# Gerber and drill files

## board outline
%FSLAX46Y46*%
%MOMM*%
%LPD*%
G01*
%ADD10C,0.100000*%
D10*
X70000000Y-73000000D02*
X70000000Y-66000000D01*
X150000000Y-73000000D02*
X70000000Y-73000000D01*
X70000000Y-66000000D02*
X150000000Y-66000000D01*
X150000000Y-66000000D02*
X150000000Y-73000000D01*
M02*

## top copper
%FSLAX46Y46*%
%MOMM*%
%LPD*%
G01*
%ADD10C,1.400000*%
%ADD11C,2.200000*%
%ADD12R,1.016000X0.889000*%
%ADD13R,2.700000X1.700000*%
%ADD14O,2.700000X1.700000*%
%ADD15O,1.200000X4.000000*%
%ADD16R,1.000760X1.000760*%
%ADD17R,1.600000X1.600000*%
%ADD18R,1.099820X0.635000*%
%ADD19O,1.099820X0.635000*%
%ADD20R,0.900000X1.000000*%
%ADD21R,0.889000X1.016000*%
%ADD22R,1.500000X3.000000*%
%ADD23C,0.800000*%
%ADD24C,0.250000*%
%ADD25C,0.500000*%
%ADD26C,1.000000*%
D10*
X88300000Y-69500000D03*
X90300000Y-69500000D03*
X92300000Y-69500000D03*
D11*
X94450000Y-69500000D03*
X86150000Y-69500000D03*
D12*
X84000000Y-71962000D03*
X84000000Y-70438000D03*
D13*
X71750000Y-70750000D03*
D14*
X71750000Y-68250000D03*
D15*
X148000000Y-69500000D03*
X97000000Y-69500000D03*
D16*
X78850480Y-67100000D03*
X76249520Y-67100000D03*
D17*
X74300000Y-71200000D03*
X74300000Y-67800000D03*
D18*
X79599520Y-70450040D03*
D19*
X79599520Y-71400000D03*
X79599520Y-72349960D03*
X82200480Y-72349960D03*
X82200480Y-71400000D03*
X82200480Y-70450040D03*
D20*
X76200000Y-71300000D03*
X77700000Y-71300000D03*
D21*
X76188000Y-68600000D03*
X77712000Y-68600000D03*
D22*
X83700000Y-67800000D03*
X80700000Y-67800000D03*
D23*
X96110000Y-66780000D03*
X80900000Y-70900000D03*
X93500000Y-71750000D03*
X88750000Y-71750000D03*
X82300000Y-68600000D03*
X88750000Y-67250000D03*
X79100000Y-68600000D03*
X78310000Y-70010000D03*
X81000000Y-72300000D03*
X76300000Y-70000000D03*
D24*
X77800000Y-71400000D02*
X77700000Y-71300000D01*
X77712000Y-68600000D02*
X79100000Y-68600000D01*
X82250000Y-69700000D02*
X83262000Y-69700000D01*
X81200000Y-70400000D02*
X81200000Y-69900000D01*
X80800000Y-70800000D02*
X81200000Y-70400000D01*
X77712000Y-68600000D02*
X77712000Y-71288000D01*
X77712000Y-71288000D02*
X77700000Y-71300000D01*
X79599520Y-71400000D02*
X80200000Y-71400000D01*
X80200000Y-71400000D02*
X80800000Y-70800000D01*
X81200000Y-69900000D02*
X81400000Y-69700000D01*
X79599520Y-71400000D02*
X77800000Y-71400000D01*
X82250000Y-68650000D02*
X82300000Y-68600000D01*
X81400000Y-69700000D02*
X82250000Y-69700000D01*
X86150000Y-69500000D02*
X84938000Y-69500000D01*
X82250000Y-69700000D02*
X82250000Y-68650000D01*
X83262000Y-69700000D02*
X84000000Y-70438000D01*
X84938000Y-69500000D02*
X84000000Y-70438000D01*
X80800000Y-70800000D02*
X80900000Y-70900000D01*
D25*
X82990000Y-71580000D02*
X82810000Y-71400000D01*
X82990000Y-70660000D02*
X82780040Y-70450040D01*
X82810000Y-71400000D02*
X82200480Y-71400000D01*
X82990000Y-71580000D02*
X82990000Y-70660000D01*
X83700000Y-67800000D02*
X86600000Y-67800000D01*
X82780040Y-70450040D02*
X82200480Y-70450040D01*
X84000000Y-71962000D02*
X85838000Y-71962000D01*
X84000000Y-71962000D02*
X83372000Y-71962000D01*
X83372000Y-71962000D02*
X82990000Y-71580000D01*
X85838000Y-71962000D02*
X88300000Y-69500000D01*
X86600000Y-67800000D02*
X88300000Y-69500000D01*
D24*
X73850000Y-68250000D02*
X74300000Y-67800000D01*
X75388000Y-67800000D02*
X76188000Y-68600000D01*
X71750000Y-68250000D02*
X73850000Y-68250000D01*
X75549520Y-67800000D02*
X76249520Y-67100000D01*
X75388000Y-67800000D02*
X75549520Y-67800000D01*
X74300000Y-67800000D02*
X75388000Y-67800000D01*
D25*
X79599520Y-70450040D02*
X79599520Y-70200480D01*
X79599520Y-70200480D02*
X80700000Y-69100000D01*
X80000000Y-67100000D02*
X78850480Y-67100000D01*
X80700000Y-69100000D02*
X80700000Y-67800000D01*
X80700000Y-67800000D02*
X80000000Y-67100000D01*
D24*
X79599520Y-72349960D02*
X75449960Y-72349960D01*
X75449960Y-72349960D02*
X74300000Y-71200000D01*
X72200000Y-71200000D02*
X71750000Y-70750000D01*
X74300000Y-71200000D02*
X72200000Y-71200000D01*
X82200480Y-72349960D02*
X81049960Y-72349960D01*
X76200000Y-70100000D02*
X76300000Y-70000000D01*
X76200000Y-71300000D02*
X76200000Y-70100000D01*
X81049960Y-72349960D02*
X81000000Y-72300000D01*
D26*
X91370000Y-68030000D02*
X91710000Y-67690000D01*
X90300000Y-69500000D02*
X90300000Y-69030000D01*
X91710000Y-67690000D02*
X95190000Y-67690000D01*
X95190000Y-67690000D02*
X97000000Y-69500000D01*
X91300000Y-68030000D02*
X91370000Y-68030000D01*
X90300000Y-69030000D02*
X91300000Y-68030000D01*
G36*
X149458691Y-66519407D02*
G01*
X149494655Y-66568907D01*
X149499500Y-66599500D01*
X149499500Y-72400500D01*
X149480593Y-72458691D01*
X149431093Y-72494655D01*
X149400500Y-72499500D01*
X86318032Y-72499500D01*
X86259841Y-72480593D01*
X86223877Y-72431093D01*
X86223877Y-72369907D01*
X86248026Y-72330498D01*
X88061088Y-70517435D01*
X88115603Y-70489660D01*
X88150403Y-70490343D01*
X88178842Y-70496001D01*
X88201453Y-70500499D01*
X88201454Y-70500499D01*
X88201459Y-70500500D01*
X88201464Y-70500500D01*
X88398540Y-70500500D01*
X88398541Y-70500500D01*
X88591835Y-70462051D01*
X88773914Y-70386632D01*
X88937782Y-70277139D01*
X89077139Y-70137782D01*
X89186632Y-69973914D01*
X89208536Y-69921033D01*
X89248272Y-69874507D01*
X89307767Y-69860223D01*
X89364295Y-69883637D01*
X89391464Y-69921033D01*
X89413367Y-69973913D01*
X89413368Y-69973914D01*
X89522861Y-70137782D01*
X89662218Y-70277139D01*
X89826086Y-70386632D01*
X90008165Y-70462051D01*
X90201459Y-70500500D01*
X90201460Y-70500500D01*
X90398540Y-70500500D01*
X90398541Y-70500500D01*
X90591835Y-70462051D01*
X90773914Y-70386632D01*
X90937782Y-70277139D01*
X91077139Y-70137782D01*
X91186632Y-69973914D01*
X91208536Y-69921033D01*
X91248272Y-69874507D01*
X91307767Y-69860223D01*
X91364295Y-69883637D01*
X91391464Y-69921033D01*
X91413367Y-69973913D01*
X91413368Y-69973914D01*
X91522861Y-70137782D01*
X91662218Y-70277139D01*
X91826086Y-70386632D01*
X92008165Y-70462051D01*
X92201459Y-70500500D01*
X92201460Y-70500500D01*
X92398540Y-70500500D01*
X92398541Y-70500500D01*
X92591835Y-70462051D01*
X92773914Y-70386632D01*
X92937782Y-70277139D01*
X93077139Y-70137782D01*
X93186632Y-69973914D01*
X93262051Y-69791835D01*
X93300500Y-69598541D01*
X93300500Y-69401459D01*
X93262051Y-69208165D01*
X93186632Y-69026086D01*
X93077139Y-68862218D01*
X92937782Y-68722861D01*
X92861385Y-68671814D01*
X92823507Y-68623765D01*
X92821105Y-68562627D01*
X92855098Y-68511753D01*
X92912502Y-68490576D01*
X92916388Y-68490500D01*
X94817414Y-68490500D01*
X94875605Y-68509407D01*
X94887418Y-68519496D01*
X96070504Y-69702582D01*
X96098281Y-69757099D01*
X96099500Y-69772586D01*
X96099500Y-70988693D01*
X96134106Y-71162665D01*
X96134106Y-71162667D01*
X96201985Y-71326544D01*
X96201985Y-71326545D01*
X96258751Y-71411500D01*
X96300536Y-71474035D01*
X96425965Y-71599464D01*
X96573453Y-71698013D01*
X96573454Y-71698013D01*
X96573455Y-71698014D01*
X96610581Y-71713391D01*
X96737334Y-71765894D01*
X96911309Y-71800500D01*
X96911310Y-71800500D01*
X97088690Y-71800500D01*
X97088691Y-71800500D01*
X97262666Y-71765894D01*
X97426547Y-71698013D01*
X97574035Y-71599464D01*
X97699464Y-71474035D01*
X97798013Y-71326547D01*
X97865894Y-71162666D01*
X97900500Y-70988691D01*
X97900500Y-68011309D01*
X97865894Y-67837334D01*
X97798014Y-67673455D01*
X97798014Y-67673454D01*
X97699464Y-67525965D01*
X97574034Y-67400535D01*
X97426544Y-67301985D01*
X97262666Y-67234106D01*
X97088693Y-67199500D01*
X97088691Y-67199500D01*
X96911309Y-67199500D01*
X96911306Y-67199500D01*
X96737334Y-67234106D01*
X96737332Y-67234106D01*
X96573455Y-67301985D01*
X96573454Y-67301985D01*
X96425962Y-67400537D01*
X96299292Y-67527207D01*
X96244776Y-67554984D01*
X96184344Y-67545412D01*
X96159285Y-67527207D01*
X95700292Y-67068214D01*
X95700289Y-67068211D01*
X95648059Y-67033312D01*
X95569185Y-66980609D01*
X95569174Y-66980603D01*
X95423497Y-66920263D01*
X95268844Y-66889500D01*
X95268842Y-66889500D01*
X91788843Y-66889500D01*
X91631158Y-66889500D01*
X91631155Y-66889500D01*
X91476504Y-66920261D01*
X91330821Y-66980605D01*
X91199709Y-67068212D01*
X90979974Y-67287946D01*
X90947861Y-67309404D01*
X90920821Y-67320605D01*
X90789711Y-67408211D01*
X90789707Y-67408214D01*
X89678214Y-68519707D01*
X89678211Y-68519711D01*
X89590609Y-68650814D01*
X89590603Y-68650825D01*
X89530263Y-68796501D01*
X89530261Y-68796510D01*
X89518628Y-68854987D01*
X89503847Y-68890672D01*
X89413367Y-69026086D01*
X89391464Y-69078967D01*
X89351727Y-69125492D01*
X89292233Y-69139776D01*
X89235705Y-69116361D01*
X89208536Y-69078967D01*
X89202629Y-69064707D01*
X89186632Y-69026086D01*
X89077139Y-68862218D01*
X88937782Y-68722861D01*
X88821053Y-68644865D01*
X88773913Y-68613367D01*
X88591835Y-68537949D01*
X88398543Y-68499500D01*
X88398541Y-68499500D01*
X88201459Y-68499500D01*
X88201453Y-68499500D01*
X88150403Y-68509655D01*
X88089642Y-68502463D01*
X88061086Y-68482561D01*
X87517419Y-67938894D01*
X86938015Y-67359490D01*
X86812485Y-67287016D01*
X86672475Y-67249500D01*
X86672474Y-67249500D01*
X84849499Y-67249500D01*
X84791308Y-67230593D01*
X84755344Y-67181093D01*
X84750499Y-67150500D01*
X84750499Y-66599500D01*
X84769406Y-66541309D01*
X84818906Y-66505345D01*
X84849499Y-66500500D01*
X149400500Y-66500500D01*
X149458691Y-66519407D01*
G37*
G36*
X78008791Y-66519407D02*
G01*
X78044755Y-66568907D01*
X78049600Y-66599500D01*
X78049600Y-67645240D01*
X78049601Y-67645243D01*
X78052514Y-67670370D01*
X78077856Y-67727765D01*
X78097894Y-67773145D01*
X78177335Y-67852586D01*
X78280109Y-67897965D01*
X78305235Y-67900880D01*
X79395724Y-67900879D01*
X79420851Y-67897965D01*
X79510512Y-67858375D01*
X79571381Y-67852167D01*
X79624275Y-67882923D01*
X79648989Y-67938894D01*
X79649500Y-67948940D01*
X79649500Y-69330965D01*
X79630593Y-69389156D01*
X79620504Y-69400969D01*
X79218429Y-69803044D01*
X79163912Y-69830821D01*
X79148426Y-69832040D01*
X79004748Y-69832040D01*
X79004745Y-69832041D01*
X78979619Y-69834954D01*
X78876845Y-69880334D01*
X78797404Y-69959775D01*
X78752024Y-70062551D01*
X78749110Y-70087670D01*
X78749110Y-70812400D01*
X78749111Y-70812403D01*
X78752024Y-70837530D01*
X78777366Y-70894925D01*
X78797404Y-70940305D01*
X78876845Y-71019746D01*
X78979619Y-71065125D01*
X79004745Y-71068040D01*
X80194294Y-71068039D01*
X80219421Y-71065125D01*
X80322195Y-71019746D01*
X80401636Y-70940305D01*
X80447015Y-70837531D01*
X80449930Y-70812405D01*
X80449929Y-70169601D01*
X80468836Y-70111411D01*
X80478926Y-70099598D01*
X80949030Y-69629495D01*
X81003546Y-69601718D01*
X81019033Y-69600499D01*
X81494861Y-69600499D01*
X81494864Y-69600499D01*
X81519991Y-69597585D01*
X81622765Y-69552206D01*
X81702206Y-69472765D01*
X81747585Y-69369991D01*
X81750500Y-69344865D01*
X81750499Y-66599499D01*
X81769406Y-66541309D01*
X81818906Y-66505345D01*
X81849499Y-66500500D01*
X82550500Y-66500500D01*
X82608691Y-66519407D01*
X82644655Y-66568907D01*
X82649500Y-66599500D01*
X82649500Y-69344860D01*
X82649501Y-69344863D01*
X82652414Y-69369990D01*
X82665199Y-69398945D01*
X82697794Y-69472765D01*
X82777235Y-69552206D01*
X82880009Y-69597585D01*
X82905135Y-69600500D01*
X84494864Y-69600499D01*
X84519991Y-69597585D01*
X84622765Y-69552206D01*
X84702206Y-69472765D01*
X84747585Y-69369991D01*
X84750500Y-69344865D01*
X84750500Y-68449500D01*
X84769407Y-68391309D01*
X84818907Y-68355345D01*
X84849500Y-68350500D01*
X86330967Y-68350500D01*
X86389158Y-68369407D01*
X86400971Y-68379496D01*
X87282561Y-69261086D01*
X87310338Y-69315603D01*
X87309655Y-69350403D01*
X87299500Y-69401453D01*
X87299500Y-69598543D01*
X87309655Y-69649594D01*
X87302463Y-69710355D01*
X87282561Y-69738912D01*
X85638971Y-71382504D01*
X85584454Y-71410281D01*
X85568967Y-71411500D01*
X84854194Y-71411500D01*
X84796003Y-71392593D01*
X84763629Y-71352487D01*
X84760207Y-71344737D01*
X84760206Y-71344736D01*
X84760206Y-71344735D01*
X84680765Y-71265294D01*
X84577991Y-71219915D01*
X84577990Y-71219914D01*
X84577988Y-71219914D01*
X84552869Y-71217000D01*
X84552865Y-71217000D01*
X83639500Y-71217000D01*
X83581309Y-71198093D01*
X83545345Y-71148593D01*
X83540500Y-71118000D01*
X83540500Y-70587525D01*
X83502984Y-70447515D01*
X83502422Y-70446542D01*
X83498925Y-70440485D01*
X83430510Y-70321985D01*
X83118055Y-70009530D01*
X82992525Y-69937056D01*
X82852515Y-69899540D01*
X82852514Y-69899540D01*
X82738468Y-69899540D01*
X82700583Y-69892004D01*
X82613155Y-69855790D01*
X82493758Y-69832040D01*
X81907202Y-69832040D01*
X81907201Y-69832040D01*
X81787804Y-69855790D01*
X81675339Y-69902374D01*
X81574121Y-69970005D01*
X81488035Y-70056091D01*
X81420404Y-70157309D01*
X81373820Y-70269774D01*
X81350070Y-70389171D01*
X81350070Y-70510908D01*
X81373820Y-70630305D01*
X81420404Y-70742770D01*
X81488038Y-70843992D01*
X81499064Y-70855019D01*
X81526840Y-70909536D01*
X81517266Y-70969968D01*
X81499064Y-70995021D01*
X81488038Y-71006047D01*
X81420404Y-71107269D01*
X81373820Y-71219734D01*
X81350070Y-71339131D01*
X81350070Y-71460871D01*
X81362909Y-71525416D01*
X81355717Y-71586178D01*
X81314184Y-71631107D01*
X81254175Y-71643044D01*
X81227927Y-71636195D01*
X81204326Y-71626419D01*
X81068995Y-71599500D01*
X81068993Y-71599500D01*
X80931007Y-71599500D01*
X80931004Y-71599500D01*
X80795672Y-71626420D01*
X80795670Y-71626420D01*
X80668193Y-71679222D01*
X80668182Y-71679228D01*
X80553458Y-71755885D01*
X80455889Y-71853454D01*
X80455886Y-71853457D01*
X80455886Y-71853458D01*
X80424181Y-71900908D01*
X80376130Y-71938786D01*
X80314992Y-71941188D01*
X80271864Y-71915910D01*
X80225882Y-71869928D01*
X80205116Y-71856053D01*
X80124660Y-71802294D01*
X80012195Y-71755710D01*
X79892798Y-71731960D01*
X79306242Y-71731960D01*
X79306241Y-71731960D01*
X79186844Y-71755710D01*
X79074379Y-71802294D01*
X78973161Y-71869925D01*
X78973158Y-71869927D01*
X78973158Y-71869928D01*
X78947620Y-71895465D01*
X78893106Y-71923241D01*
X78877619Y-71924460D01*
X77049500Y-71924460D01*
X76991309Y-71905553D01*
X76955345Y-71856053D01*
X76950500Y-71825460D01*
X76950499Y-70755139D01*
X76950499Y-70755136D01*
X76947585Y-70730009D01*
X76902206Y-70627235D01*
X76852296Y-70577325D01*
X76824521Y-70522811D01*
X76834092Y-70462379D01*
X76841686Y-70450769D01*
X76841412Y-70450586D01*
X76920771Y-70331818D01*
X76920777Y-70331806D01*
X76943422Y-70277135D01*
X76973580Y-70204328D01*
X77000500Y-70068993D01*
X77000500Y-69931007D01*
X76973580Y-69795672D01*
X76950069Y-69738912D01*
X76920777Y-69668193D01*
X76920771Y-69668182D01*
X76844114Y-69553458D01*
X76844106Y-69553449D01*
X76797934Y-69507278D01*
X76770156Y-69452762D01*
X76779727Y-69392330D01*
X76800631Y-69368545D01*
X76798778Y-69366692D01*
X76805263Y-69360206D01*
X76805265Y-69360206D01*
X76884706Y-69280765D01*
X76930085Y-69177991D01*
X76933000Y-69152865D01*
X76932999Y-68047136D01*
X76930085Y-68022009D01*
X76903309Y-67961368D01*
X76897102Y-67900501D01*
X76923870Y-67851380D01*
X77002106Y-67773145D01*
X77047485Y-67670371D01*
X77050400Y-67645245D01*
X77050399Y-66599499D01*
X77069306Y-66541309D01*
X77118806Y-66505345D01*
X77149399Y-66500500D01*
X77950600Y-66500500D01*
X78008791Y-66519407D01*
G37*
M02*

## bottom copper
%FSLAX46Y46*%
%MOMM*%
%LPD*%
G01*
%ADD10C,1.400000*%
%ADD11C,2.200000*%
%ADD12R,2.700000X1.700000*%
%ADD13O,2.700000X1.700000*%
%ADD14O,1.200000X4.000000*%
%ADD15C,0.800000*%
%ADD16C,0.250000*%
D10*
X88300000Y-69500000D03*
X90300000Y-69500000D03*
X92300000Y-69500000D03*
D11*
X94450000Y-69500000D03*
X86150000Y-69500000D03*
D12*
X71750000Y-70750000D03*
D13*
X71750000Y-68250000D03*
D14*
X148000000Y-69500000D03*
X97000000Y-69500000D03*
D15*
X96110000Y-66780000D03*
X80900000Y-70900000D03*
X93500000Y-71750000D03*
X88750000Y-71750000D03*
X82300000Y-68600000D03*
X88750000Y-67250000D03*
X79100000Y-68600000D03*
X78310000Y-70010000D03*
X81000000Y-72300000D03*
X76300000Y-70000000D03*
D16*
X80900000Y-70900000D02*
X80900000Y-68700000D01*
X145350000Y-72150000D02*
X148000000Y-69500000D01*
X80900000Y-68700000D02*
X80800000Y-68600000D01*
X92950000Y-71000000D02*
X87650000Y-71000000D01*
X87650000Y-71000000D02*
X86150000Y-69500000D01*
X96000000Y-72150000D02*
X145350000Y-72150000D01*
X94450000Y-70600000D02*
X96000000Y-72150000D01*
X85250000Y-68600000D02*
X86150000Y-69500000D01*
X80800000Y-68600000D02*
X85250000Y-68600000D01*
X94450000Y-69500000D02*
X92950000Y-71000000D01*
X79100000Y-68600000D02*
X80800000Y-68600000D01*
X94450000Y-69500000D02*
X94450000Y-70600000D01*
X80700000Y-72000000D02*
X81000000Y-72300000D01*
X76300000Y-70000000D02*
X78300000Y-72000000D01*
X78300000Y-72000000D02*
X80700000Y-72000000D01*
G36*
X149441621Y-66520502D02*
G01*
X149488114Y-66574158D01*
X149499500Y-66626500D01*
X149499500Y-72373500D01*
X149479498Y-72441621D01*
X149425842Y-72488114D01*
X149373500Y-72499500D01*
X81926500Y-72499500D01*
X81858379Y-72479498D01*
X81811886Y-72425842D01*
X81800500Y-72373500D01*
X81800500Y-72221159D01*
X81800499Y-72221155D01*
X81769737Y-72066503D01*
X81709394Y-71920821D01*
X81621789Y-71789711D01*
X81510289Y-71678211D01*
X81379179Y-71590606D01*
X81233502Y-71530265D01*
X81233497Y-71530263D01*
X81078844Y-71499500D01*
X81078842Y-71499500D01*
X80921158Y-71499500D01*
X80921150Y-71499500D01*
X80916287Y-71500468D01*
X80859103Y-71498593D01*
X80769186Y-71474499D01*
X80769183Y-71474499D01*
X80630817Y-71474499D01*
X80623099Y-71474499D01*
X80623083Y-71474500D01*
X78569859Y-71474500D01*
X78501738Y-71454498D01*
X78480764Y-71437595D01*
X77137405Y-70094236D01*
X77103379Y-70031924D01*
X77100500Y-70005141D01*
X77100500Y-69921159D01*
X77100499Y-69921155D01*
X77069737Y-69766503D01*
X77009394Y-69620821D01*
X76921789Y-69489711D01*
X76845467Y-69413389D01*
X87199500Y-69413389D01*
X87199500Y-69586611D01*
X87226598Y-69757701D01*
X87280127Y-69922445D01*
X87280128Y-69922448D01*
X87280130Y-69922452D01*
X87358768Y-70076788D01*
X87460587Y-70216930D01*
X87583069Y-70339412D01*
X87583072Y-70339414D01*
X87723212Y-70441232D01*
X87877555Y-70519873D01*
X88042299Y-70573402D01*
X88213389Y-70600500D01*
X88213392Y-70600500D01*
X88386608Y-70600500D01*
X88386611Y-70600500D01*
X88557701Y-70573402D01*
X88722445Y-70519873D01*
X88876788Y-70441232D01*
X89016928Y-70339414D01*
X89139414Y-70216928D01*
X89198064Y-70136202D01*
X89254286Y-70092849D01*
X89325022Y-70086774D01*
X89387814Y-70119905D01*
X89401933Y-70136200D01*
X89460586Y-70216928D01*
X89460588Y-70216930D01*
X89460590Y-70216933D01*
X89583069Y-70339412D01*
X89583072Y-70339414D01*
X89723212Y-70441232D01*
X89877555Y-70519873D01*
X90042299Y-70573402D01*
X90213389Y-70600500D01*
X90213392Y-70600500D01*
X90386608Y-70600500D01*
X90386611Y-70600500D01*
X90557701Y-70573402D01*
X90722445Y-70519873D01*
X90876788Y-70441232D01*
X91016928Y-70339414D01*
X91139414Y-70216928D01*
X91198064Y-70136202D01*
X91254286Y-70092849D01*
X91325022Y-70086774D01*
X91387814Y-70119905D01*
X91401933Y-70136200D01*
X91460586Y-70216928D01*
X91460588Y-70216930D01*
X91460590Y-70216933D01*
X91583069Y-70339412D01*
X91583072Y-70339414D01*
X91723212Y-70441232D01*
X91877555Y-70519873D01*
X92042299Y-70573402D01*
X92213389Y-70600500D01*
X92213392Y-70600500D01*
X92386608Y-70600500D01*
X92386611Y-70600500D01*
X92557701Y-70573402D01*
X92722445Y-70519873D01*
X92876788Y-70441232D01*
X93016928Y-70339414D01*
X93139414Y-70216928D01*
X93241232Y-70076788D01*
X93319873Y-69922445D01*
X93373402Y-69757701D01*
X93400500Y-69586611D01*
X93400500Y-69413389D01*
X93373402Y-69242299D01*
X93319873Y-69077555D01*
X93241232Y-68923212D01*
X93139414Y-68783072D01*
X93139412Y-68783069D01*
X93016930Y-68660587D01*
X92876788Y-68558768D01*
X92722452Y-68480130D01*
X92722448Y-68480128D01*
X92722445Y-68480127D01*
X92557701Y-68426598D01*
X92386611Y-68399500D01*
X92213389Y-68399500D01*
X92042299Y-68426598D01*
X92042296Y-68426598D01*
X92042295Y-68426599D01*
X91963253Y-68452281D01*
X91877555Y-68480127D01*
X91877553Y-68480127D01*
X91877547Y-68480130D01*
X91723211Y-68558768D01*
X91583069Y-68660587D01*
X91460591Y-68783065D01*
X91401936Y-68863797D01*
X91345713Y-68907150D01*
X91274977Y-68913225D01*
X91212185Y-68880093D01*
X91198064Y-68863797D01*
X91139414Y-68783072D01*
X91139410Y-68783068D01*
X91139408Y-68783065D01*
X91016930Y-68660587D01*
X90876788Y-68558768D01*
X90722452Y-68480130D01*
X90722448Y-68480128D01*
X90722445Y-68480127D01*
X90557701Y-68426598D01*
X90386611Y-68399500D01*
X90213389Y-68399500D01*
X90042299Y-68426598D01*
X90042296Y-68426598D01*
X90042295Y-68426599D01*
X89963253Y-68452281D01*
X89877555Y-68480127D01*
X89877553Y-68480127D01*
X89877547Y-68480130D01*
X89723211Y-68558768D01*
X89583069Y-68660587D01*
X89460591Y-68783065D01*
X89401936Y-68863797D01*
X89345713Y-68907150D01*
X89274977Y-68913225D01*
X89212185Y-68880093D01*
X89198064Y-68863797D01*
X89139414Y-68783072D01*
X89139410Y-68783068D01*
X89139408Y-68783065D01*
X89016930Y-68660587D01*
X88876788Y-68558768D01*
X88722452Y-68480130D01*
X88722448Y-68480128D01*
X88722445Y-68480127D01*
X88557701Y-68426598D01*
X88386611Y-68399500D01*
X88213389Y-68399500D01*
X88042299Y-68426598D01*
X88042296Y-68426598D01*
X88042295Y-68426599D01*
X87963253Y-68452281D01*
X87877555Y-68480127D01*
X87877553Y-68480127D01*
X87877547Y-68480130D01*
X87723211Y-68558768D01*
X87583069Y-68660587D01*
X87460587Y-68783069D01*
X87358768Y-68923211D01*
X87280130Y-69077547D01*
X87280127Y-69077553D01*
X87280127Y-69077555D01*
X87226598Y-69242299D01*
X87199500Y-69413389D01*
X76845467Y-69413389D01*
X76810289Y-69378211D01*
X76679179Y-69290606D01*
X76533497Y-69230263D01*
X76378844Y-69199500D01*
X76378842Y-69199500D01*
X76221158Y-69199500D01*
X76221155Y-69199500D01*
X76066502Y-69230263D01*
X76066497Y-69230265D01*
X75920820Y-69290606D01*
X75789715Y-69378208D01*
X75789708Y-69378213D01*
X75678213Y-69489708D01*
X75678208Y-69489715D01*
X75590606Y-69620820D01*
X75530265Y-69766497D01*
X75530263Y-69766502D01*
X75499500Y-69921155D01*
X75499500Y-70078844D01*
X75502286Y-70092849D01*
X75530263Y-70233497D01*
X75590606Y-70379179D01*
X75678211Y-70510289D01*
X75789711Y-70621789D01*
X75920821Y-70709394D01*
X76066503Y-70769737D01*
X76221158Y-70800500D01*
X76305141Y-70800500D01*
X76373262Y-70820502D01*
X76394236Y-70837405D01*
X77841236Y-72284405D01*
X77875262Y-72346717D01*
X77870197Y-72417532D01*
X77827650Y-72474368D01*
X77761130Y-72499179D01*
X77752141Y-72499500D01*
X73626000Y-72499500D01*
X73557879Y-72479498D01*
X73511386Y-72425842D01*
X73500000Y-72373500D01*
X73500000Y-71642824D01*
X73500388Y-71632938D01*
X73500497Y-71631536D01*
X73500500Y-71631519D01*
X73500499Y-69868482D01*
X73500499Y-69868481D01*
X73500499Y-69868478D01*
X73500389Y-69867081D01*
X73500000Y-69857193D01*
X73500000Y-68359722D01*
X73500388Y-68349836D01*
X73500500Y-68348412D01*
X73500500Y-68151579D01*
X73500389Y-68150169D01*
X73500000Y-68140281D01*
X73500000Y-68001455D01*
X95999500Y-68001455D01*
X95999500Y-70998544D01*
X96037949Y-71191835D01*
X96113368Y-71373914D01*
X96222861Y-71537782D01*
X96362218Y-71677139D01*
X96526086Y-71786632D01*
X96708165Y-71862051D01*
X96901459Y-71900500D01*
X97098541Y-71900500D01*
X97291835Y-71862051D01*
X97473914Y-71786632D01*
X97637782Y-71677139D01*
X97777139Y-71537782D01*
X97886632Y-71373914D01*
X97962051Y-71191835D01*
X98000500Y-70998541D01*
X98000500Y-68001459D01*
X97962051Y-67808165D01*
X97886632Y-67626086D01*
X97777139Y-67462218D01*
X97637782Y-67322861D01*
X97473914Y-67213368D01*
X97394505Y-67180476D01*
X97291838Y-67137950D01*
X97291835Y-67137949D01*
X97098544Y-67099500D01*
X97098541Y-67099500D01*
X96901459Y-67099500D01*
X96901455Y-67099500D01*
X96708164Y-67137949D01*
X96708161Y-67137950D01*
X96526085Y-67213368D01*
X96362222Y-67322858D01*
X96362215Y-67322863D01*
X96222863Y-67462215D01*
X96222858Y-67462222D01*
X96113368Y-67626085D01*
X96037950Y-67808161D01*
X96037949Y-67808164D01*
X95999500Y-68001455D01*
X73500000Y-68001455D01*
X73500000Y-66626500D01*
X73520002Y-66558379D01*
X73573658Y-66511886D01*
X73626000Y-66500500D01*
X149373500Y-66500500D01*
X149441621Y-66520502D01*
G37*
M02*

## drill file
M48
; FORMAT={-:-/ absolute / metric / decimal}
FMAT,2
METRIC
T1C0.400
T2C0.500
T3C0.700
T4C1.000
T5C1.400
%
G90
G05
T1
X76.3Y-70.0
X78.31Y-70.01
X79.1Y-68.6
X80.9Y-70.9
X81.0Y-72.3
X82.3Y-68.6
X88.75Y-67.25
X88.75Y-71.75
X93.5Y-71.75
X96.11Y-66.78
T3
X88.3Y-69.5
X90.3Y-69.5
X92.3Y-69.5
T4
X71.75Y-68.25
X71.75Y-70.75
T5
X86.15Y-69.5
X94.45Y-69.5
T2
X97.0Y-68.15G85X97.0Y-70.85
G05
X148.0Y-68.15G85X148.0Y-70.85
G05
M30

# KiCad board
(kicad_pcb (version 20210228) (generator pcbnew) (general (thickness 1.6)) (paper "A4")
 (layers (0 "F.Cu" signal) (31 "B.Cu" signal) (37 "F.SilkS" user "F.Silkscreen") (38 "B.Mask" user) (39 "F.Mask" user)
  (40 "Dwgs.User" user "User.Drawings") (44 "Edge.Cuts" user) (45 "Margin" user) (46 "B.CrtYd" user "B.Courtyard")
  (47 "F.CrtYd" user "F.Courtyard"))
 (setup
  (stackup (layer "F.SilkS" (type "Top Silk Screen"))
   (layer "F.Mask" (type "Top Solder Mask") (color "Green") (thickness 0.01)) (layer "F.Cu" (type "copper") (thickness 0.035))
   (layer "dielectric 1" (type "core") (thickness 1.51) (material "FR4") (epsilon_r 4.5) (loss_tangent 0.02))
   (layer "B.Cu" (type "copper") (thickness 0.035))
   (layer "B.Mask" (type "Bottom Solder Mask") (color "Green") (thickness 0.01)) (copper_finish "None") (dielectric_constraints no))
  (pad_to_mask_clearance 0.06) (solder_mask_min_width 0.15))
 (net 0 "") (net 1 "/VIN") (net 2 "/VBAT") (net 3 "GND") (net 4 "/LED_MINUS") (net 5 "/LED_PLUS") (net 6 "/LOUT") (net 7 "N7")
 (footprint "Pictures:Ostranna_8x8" (layer "F.Cu") (at 103.36 69.7)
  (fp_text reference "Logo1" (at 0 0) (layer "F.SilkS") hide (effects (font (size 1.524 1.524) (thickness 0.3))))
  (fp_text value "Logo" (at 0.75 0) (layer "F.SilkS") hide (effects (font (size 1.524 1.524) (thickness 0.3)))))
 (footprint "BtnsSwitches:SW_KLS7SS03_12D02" (layer "F.Cu") (at 90.3 69.5)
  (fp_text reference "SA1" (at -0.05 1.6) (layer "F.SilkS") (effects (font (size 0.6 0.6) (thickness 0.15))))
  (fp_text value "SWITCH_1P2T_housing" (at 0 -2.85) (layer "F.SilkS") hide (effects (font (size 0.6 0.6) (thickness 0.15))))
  (pad "1" thru_hole circle (at -2 0) (locked) (size 1.4 1.4) (drill 0.7) (layers *.Cu *.Mask) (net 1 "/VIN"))
  (pad "2" thru_hole circle (at 0 0) (locked) (size 1.4 1.4) (drill 0.7) (layers *.Cu *.Mask) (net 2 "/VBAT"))
  (pad "3" thru_hole circle (at 2 0) (locked) (size 1.4 1.4) (drill 0.7) (layers *.Cu *.Mask))
  (pad "H" thru_hole circle (at 4.15 0) (locked) (size 2.2 2.2) (drill 1.4) (layers *.Cu *.Mask) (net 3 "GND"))
  (pad "H" thru_hole circle (at -4.15 0) (locked) (size 2.2 2.2) (drill 1.4) (layers *.Cu *.Mask) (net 3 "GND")))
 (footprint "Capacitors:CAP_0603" (layer "F.Cu") (at 84 71.2 90)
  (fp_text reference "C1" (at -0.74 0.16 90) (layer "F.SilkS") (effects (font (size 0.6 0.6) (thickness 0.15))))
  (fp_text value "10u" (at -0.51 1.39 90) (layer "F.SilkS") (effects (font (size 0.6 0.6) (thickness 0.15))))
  (pad "1" smd rect (at -0.762 0 90) (locked) (size 0.889 1.016) (layers "F.Cu" "F.Paste" "F.Mask") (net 1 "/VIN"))
  (pad "2" smd rect (at 0.762 0 90) (locked) (size 0.889 1.016) (layers "F.Cu" "F.Paste" "F.Mask") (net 3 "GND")))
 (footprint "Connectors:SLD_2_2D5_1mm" (layer "F.Cu") (at 71.75 69.5 90)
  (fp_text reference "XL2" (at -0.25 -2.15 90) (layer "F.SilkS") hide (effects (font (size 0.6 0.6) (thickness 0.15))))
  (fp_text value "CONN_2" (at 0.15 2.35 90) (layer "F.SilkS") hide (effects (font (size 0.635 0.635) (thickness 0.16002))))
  (pad "1" thru_hole rect (at -1.25 0 90) (locked) (size 1.7 2.7) (drill 1) (layers *.Cu *.Mask) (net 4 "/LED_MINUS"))
  (pad "2" thru_hole oval (at 1.25 0 90) (locked) (size 1.7 2.7) (drill 1) (layers *.Cu *.Mask) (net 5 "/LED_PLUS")))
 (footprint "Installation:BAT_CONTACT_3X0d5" (layer "F.Cu") (at 148 69.5)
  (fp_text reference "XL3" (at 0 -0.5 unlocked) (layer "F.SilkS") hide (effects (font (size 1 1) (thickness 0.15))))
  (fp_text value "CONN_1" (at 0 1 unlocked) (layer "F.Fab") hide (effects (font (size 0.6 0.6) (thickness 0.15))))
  (pad "1" thru_hole oval (at 0 0) (locked) (size 1.2 4) (drill oval 0.5 3.2) (layers *.Cu *.Mask) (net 3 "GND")))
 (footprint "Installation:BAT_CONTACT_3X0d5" (layer "F.Cu") (at 97 69.5)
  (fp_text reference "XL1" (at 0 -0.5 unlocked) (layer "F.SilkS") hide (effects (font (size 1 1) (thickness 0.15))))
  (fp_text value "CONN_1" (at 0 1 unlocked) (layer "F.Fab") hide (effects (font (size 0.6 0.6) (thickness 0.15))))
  (pad "1" thru_hole oval (at 0 0) (locked) (size 1.2 4) (drill oval 0.5 3.2) (layers *.Cu *.Mask) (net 2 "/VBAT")))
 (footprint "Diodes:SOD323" (layer "F.Cu") (at 77.55 67.1)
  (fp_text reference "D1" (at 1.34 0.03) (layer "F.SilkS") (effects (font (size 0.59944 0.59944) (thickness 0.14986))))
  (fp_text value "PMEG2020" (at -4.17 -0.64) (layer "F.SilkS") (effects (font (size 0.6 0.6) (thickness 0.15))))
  (pad "A" smd rect (at 1.30048 0) (locked) (size 1.00076 1.00076) (layers "F.Cu" "F.Paste" "F.Mask") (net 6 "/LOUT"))
  (pad "C" smd rect (at -1.30048 0) (locked) (size 1.00076 1.00076) (layers "F.Cu" "F.Paste" "F.Mask") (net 5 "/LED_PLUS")))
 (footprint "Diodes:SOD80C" (layer "F.Cu") (at 74.3 69.5 -90)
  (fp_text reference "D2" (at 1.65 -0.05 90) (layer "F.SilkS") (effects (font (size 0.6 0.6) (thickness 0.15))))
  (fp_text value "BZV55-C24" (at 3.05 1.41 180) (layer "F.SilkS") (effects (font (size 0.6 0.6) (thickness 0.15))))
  (pad "A" smd rect (at 1.7 0 270) (locked) (size 1.6 1.6) (layers "F.Cu" "F.Paste" "F.Mask") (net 4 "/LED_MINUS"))
  (pad "C" smd rect (at -1.7 0 270) (locked) (size 1.6 1.6) (layers "F.Cu" "F.Paste" "F.Mask") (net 5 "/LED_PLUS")))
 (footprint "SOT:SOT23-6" (layer "F.Cu") (at 80.9 71.4 -90)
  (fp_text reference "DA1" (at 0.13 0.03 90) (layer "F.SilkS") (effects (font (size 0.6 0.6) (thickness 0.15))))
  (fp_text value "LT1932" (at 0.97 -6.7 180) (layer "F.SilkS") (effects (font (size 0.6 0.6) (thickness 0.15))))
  (pad "1" smd rect (at -0.94996 1.30048 270) (locked) (size 0.635 1.09982) (layers "F.Cu" "F.Paste" "F.Mask") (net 6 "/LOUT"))
  (pad "2" smd oval (at 0 1.30048 270) (locked) (size 0.635 1.09982) (layers "F.Cu" "F.Paste" "F.Mask") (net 3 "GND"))
  (pad "3" smd oval (at 0.94996 1.30048 270) (locked) (size 0.635 1.09982) (layers "F.Cu" "F.Paste" "F.Mask") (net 4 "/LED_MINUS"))
  (pad "4" smd oval (at 0.94996 -1.30048 270) (locked) (size 0.635 1.09982) (layers "F.Cu" "F.Paste" "F.Mask") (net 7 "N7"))
  (pad "5" smd oval (at 0 -1.30048 270) (locked) (size 0.635 1.09982) (layers "F.Cu" "F.Paste" "F.Mask") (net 1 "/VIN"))
  (pad "6" smd oval (at -0.94996 -1.30048 270) (locked) (size 0.635 1.09982) (layers "F.Cu" "F.Paste" "F.Mask") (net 1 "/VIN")))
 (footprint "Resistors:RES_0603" (layer "F.Cu") (at 76.95 71.3)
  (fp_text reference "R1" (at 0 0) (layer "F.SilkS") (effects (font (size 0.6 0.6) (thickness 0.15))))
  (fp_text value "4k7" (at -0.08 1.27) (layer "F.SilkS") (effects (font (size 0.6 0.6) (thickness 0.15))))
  (pad "1" smd rect (at -0.75 0) (locked) (size 0.9 1) (layers "F.Cu" "F.Paste" "F.Mask") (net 7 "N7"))
  (pad "2" smd rect (at 0.75 0) (locked) (size 0.9 1) (layers "F.Cu" "F.Paste" "F.Mask") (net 3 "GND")))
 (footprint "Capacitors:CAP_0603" (layer "F.Cu") (at 76.95 68.6)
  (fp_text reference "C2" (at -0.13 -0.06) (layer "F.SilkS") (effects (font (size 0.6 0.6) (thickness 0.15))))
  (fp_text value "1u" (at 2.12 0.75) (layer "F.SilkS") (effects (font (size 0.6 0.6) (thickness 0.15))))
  (pad "1" smd rect (at -0.762 0) (locked) (size 0.889 1.016) (layers "F.Cu" "F.Paste" "F.Mask") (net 5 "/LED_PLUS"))
  (pad "2" smd rect (at 0.762 0) (locked) (size 0.889 1.016) (layers "F.Cu" "F.Paste" "F.Mask") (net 3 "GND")))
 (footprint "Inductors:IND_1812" (layer "F.Cu") (at 82.2 67.8 180)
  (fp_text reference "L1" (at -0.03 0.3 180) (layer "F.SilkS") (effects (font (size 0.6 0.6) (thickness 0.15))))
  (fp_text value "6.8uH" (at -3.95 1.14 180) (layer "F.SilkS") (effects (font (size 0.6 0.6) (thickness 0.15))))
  (pad "1" smd rect (at -1.5 0 180) (size 1.5 3) (layers "F.Cu" "F.Paste" "F.Mask") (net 1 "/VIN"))
  (pad "2" smd rect (at 1.5 0 180) (locked) (size 1.5 3) (layers "F.Cu" "F.Paste" "F.Mask") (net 6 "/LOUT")))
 (gr_line (start 70 73) (end 70 66) (layer "Edge.Cuts") (width 0.1))
 (gr_line (start 150 73) (end 70 73) (layer "Edge.Cuts") (width 0.1))
 (gr_line (start 70 66) (end 150 66) (layer "Edge.Cuts") (width 0.1))
 (gr_line (start 150 66) (end 150 73) (layer "Edge.Cuts") (width 0.1))
 (segment (start 77.8 71.4) (end 77.7 71.3) (width 0.25) (layer "F.Cu") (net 3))
 (segment (start 77.712 68.6) (end 79.1 68.6) (width 0.25) (layer "F.Cu") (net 3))
 (segment (start 82.25 69.7) (end 83.262 69.7) (width 0.25) (layer "F.Cu") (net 3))
 (segment (start 81.2 70.4) (end 81.2 69.9) (width 0.25) (layer "F.Cu") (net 3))
 (segment (start 80.8 70.8) (end 81.2 70.4) (width 0.25) (layer "F.Cu") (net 3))
 (segment (start 77.712 68.6) (end 77.712 71.288) (width 0.25) (layer "F.Cu") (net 3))
 (segment (start 77.712 71.288) (end 77.7 71.3) (width 0.25) (layer "F.Cu") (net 3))
 (segment (start 79.59952 71.4) (end 80.2 71.4) (width 0.25) (layer "F.Cu") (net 3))
 (segment (start 80.2 71.4) (end 80.8 70.8) (width 0.25) (layer "F.Cu") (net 3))
 (segment (start 81.2 69.9) (end 81.4 69.7) (width 0.25) (layer "F.Cu") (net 3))
 (segment (start 79.59952 71.4) (end 77.8 71.4) (width 0.25) (layer "F.Cu") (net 3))
 (segment (start 82.25 68.65) (end 82.3 68.6) (width 0.25) (layer "F.Cu") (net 3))
 (segment (start 81.4 69.7) (end 82.25 69.7) (width 0.25) (layer "F.Cu") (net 3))
 (segment (start 86.15 69.5) (end 84.938 69.5) (width 0.25) (layer "F.Cu") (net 3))
 (segment (start 82.25 69.7) (end 82.25 68.65) (width 0.25) (layer "F.Cu") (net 3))
 (segment (start 83.262 69.7) (end 84 70.438) (width 0.25) (layer "F.Cu") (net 3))
 (segment (start 84.938 69.5) (end 84 70.438) (width 0.25) (layer "F.Cu") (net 3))
 (segment (start 80.8 70.8) (end 80.9 70.9) (width 0.25) (layer "F.Cu") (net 3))
 (via (at 96.11 66.78) (size 0.8) (drill 0.4) (layers "F.Cu" "B.Cu") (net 3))
 (via (at 80.9 70.9) (size 0.8) (drill 0.4) (layers "F.Cu" "B.Cu") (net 3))
 (via (at 93.5 71.75) (size 0.8) (drill 0.4) (layers "F.Cu" "B.Cu") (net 3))
 (via (at 88.75 71.75) (size 0.8) (drill 0.4) (layers "F.Cu" "B.Cu") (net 3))
 (via (at 82.3 68.6) (size 0.8) (drill 0.4) (layers "F.Cu" "B.Cu") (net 3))
 (via (at 88.75 67.25) (size 0.8) (drill 0.4) (layers "F.Cu" "B.Cu") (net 3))
 (via (at 79.1 68.6) (size 0.8) (drill 0.4) (layers "F.Cu" "B.Cu") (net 3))
 (via (at 78.31 70.01) (size 0.8) (drill 0.4) (layers "F.Cu" "B.Cu") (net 3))
 (segment (start 80.9 70.9) (end 80.9 68.7) (width 0.25) (layer "B.Cu") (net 3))
 (segment (start 145.35 72.15) (end 148 69.5) (width 0.25) (layer "B.Cu") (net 3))
 (segment (start 80.9 68.7) (end 80.8 68.6) (width 0.25) (layer "B.Cu") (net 3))
 (segment (start 92.95 71) (end 87.65 71) (width 0.25) (layer "B.Cu") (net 3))
 (segment (start 87.65 71) (end 86.15 69.5) (width 0.25) (layer "B.Cu") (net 3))
 (segment (start 96 72.15) (end 145.35 72.15) (width 0.25) (layer "B.Cu") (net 3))
 (segment (start 94.45 70.6) (end 96 72.15) (width 0.25) (layer "B.Cu") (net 3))
 (segment (start 85.25 68.6) (end 86.15 69.5) (width 0.25) (layer "B.Cu") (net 3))
 (segment (start 80.8 68.6) (end 85.25 68.6) (width 0.25) (layer "B.Cu") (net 3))
 (segment (start 94.45 69.5) (end 92.95 71) (width 0.25) (layer "B.Cu") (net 3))
 (segment (start 79.1 68.6) (end 80.8 68.6) (width 0.25) (layer "B.Cu") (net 3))
 (segment (start 94.45 69.5) (end 94.45 70.6) (width 0.25) (layer "B.Cu") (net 3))
 (segment (start 82.99 71.58) (end 82.81 71.4) (width 0.5) (layer "F.Cu") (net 1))
 (segment (start 82.99 70.66) (end 82.78004 70.45004) (width 0.5) (layer "F.Cu") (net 1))
 (segment (start 82.81 71.4) (end 82.20048 71.4) (width 0.5) (layer "F.Cu") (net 1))
 (segment (start 82.99 71.58) (end 82.99 70.66) (width 0.5) (layer "F.Cu") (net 1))
 (segment (start 83.7 67.8) (end 86.6 67.8) (width 0.5) (layer "F.Cu") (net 1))
 (segment (start 82.78004 70.45004) (end 82.20048 70.45004) (width 0.5) (layer "F.Cu") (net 1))
 (segment (start 84 71.962) (end 85.838 71.962) (width 0.5) (layer "F.Cu") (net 1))
 (segment (start 84 71.962) (end 83.372 71.962) (width 0.5) (layer "F.Cu") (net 1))
 (segment (start 83.372 71.962) (end 82.99 71.58) (width 0.5) (layer "F.Cu") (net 1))
 (segment (start 85.838 71.962) (end 88.3 69.5) (width 0.5) (layer "F.Cu") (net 1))
 (segment (start 86.6 67.8) (end 88.3 69.5) (width 0.5) (layer "F.Cu") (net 1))
 (segment (start 73.85 68.25) (end 74.3 67.8) (width 0.25) (layer "F.Cu") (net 5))
 (segment (start 75.388 67.8) (end 76.188 68.6) (width 0.25) (layer "F.Cu") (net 5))
 (segment (start 71.75 68.25) (end 73.85 68.25) (width 0.25) (layer "F.Cu") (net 5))
 (segment (start 75.54952 67.8) (end 76.24952 67.1) (width 0.25) (layer "F.Cu") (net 5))
 (segment (start 75.388 67.8) (end 75.54952 67.8) (width 0.25) (layer "F.Cu") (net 5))
 (segment (start 74.3 67.8) (end 75.388 67.8) (width 0.25) (layer "F.Cu") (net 5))
 (segment (start 79.59952 70.45004) (end 79.59952 70.20048) (width 0.5) (layer "F.Cu") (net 6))
 (segment (start 79.59952 70.20048) (end 80.7 69.1) (width 0.5) (layer "F.Cu") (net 6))
 (segment (start 80 67.1) (end 78.85048 67.1) (width 0.5) (layer "F.Cu") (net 6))
 (segment (start 80.7 69.1) (end 80.7 67.8) (width 0.5) (layer "F.Cu") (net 6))
 (segment (start 80.7 67.8) (end 80 67.1) (width 0.5) (layer "F.Cu") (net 6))
 (segment (start 79.59952 72.34996) (end 75.44996 72.34996) (width 0.25) (layer "F.Cu") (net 4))
 (segment (start 75.44996 72.34996) (end 74.3 71.2) (width 0.25) (layer "F.Cu") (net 4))
 (segment (start 72.2 71.2) (end 71.75 70.75) (width 0.25) (layer "F.Cu") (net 4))
 (segment (start 74.3 71.2) (end 72.2 71.2) (width 0.25) (layer "F.Cu") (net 4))
 (segment (start 82.20048 72.34996) (end 81.04996 72.34996) (width 0.25) (layer "F.Cu") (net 7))
 (segment (start 76.2 70.1) (end 76.3 70) (width 0.25) (layer "F.Cu") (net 7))
 (segment (start 76.2 71.3) (end 76.2 70.1) (width 0.25) (layer "F.Cu") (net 7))
 (segment (start 81.04996 72.34996) (end 81 72.3) (width 0.25) (layer "F.Cu") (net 7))
 (via (at 81 72.3) (size 0.8) (drill 0.4) (layers "F.Cu" "B.Cu") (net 7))
 (via (at 76.3 70) (size 0.8) (drill 0.4) (layers "F.Cu" "B.Cu") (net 7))
 (segment (start 80.7 72) (end 81 72.3) (width 0.25) (layer "B.Cu") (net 7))
 (segment (start 76.3 70) (end 78.3 72) (width 0.25) (layer "B.Cu") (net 7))
 (segment (start 78.3 72) (end 80.7 72) (width 0.25) (layer "B.Cu") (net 7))
 (segment (start 91.37 68.03) (end 91.71 67.69) (width 1) (layer "F.Cu") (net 2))
 (segment (start 90.3 69.5) (end 90.3 69.03) (width 1) (layer "F.Cu") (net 2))
 (segment (start 91.71 67.69) (end 95.19 67.69) (width 1) (layer "F.Cu") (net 2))
 (segment (start 95.19 67.69) (end 97 69.5) (width 1) (layer "F.Cu") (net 2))
 (segment (start 91.3 68.03) (end 91.37 68.03) (width 1) (layer "F.Cu") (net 2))
 (segment (start 90.3 69.03) (end 91.3 68.03) (width 1) (layer "F.Cu") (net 2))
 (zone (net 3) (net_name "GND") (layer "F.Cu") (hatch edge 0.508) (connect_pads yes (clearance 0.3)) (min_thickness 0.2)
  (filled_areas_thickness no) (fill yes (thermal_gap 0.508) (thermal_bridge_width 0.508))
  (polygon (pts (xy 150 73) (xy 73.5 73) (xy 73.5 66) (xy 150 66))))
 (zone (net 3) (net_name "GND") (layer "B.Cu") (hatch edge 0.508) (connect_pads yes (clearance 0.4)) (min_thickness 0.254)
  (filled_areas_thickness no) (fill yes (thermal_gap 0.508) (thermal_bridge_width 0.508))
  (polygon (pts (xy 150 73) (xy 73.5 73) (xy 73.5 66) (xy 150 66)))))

